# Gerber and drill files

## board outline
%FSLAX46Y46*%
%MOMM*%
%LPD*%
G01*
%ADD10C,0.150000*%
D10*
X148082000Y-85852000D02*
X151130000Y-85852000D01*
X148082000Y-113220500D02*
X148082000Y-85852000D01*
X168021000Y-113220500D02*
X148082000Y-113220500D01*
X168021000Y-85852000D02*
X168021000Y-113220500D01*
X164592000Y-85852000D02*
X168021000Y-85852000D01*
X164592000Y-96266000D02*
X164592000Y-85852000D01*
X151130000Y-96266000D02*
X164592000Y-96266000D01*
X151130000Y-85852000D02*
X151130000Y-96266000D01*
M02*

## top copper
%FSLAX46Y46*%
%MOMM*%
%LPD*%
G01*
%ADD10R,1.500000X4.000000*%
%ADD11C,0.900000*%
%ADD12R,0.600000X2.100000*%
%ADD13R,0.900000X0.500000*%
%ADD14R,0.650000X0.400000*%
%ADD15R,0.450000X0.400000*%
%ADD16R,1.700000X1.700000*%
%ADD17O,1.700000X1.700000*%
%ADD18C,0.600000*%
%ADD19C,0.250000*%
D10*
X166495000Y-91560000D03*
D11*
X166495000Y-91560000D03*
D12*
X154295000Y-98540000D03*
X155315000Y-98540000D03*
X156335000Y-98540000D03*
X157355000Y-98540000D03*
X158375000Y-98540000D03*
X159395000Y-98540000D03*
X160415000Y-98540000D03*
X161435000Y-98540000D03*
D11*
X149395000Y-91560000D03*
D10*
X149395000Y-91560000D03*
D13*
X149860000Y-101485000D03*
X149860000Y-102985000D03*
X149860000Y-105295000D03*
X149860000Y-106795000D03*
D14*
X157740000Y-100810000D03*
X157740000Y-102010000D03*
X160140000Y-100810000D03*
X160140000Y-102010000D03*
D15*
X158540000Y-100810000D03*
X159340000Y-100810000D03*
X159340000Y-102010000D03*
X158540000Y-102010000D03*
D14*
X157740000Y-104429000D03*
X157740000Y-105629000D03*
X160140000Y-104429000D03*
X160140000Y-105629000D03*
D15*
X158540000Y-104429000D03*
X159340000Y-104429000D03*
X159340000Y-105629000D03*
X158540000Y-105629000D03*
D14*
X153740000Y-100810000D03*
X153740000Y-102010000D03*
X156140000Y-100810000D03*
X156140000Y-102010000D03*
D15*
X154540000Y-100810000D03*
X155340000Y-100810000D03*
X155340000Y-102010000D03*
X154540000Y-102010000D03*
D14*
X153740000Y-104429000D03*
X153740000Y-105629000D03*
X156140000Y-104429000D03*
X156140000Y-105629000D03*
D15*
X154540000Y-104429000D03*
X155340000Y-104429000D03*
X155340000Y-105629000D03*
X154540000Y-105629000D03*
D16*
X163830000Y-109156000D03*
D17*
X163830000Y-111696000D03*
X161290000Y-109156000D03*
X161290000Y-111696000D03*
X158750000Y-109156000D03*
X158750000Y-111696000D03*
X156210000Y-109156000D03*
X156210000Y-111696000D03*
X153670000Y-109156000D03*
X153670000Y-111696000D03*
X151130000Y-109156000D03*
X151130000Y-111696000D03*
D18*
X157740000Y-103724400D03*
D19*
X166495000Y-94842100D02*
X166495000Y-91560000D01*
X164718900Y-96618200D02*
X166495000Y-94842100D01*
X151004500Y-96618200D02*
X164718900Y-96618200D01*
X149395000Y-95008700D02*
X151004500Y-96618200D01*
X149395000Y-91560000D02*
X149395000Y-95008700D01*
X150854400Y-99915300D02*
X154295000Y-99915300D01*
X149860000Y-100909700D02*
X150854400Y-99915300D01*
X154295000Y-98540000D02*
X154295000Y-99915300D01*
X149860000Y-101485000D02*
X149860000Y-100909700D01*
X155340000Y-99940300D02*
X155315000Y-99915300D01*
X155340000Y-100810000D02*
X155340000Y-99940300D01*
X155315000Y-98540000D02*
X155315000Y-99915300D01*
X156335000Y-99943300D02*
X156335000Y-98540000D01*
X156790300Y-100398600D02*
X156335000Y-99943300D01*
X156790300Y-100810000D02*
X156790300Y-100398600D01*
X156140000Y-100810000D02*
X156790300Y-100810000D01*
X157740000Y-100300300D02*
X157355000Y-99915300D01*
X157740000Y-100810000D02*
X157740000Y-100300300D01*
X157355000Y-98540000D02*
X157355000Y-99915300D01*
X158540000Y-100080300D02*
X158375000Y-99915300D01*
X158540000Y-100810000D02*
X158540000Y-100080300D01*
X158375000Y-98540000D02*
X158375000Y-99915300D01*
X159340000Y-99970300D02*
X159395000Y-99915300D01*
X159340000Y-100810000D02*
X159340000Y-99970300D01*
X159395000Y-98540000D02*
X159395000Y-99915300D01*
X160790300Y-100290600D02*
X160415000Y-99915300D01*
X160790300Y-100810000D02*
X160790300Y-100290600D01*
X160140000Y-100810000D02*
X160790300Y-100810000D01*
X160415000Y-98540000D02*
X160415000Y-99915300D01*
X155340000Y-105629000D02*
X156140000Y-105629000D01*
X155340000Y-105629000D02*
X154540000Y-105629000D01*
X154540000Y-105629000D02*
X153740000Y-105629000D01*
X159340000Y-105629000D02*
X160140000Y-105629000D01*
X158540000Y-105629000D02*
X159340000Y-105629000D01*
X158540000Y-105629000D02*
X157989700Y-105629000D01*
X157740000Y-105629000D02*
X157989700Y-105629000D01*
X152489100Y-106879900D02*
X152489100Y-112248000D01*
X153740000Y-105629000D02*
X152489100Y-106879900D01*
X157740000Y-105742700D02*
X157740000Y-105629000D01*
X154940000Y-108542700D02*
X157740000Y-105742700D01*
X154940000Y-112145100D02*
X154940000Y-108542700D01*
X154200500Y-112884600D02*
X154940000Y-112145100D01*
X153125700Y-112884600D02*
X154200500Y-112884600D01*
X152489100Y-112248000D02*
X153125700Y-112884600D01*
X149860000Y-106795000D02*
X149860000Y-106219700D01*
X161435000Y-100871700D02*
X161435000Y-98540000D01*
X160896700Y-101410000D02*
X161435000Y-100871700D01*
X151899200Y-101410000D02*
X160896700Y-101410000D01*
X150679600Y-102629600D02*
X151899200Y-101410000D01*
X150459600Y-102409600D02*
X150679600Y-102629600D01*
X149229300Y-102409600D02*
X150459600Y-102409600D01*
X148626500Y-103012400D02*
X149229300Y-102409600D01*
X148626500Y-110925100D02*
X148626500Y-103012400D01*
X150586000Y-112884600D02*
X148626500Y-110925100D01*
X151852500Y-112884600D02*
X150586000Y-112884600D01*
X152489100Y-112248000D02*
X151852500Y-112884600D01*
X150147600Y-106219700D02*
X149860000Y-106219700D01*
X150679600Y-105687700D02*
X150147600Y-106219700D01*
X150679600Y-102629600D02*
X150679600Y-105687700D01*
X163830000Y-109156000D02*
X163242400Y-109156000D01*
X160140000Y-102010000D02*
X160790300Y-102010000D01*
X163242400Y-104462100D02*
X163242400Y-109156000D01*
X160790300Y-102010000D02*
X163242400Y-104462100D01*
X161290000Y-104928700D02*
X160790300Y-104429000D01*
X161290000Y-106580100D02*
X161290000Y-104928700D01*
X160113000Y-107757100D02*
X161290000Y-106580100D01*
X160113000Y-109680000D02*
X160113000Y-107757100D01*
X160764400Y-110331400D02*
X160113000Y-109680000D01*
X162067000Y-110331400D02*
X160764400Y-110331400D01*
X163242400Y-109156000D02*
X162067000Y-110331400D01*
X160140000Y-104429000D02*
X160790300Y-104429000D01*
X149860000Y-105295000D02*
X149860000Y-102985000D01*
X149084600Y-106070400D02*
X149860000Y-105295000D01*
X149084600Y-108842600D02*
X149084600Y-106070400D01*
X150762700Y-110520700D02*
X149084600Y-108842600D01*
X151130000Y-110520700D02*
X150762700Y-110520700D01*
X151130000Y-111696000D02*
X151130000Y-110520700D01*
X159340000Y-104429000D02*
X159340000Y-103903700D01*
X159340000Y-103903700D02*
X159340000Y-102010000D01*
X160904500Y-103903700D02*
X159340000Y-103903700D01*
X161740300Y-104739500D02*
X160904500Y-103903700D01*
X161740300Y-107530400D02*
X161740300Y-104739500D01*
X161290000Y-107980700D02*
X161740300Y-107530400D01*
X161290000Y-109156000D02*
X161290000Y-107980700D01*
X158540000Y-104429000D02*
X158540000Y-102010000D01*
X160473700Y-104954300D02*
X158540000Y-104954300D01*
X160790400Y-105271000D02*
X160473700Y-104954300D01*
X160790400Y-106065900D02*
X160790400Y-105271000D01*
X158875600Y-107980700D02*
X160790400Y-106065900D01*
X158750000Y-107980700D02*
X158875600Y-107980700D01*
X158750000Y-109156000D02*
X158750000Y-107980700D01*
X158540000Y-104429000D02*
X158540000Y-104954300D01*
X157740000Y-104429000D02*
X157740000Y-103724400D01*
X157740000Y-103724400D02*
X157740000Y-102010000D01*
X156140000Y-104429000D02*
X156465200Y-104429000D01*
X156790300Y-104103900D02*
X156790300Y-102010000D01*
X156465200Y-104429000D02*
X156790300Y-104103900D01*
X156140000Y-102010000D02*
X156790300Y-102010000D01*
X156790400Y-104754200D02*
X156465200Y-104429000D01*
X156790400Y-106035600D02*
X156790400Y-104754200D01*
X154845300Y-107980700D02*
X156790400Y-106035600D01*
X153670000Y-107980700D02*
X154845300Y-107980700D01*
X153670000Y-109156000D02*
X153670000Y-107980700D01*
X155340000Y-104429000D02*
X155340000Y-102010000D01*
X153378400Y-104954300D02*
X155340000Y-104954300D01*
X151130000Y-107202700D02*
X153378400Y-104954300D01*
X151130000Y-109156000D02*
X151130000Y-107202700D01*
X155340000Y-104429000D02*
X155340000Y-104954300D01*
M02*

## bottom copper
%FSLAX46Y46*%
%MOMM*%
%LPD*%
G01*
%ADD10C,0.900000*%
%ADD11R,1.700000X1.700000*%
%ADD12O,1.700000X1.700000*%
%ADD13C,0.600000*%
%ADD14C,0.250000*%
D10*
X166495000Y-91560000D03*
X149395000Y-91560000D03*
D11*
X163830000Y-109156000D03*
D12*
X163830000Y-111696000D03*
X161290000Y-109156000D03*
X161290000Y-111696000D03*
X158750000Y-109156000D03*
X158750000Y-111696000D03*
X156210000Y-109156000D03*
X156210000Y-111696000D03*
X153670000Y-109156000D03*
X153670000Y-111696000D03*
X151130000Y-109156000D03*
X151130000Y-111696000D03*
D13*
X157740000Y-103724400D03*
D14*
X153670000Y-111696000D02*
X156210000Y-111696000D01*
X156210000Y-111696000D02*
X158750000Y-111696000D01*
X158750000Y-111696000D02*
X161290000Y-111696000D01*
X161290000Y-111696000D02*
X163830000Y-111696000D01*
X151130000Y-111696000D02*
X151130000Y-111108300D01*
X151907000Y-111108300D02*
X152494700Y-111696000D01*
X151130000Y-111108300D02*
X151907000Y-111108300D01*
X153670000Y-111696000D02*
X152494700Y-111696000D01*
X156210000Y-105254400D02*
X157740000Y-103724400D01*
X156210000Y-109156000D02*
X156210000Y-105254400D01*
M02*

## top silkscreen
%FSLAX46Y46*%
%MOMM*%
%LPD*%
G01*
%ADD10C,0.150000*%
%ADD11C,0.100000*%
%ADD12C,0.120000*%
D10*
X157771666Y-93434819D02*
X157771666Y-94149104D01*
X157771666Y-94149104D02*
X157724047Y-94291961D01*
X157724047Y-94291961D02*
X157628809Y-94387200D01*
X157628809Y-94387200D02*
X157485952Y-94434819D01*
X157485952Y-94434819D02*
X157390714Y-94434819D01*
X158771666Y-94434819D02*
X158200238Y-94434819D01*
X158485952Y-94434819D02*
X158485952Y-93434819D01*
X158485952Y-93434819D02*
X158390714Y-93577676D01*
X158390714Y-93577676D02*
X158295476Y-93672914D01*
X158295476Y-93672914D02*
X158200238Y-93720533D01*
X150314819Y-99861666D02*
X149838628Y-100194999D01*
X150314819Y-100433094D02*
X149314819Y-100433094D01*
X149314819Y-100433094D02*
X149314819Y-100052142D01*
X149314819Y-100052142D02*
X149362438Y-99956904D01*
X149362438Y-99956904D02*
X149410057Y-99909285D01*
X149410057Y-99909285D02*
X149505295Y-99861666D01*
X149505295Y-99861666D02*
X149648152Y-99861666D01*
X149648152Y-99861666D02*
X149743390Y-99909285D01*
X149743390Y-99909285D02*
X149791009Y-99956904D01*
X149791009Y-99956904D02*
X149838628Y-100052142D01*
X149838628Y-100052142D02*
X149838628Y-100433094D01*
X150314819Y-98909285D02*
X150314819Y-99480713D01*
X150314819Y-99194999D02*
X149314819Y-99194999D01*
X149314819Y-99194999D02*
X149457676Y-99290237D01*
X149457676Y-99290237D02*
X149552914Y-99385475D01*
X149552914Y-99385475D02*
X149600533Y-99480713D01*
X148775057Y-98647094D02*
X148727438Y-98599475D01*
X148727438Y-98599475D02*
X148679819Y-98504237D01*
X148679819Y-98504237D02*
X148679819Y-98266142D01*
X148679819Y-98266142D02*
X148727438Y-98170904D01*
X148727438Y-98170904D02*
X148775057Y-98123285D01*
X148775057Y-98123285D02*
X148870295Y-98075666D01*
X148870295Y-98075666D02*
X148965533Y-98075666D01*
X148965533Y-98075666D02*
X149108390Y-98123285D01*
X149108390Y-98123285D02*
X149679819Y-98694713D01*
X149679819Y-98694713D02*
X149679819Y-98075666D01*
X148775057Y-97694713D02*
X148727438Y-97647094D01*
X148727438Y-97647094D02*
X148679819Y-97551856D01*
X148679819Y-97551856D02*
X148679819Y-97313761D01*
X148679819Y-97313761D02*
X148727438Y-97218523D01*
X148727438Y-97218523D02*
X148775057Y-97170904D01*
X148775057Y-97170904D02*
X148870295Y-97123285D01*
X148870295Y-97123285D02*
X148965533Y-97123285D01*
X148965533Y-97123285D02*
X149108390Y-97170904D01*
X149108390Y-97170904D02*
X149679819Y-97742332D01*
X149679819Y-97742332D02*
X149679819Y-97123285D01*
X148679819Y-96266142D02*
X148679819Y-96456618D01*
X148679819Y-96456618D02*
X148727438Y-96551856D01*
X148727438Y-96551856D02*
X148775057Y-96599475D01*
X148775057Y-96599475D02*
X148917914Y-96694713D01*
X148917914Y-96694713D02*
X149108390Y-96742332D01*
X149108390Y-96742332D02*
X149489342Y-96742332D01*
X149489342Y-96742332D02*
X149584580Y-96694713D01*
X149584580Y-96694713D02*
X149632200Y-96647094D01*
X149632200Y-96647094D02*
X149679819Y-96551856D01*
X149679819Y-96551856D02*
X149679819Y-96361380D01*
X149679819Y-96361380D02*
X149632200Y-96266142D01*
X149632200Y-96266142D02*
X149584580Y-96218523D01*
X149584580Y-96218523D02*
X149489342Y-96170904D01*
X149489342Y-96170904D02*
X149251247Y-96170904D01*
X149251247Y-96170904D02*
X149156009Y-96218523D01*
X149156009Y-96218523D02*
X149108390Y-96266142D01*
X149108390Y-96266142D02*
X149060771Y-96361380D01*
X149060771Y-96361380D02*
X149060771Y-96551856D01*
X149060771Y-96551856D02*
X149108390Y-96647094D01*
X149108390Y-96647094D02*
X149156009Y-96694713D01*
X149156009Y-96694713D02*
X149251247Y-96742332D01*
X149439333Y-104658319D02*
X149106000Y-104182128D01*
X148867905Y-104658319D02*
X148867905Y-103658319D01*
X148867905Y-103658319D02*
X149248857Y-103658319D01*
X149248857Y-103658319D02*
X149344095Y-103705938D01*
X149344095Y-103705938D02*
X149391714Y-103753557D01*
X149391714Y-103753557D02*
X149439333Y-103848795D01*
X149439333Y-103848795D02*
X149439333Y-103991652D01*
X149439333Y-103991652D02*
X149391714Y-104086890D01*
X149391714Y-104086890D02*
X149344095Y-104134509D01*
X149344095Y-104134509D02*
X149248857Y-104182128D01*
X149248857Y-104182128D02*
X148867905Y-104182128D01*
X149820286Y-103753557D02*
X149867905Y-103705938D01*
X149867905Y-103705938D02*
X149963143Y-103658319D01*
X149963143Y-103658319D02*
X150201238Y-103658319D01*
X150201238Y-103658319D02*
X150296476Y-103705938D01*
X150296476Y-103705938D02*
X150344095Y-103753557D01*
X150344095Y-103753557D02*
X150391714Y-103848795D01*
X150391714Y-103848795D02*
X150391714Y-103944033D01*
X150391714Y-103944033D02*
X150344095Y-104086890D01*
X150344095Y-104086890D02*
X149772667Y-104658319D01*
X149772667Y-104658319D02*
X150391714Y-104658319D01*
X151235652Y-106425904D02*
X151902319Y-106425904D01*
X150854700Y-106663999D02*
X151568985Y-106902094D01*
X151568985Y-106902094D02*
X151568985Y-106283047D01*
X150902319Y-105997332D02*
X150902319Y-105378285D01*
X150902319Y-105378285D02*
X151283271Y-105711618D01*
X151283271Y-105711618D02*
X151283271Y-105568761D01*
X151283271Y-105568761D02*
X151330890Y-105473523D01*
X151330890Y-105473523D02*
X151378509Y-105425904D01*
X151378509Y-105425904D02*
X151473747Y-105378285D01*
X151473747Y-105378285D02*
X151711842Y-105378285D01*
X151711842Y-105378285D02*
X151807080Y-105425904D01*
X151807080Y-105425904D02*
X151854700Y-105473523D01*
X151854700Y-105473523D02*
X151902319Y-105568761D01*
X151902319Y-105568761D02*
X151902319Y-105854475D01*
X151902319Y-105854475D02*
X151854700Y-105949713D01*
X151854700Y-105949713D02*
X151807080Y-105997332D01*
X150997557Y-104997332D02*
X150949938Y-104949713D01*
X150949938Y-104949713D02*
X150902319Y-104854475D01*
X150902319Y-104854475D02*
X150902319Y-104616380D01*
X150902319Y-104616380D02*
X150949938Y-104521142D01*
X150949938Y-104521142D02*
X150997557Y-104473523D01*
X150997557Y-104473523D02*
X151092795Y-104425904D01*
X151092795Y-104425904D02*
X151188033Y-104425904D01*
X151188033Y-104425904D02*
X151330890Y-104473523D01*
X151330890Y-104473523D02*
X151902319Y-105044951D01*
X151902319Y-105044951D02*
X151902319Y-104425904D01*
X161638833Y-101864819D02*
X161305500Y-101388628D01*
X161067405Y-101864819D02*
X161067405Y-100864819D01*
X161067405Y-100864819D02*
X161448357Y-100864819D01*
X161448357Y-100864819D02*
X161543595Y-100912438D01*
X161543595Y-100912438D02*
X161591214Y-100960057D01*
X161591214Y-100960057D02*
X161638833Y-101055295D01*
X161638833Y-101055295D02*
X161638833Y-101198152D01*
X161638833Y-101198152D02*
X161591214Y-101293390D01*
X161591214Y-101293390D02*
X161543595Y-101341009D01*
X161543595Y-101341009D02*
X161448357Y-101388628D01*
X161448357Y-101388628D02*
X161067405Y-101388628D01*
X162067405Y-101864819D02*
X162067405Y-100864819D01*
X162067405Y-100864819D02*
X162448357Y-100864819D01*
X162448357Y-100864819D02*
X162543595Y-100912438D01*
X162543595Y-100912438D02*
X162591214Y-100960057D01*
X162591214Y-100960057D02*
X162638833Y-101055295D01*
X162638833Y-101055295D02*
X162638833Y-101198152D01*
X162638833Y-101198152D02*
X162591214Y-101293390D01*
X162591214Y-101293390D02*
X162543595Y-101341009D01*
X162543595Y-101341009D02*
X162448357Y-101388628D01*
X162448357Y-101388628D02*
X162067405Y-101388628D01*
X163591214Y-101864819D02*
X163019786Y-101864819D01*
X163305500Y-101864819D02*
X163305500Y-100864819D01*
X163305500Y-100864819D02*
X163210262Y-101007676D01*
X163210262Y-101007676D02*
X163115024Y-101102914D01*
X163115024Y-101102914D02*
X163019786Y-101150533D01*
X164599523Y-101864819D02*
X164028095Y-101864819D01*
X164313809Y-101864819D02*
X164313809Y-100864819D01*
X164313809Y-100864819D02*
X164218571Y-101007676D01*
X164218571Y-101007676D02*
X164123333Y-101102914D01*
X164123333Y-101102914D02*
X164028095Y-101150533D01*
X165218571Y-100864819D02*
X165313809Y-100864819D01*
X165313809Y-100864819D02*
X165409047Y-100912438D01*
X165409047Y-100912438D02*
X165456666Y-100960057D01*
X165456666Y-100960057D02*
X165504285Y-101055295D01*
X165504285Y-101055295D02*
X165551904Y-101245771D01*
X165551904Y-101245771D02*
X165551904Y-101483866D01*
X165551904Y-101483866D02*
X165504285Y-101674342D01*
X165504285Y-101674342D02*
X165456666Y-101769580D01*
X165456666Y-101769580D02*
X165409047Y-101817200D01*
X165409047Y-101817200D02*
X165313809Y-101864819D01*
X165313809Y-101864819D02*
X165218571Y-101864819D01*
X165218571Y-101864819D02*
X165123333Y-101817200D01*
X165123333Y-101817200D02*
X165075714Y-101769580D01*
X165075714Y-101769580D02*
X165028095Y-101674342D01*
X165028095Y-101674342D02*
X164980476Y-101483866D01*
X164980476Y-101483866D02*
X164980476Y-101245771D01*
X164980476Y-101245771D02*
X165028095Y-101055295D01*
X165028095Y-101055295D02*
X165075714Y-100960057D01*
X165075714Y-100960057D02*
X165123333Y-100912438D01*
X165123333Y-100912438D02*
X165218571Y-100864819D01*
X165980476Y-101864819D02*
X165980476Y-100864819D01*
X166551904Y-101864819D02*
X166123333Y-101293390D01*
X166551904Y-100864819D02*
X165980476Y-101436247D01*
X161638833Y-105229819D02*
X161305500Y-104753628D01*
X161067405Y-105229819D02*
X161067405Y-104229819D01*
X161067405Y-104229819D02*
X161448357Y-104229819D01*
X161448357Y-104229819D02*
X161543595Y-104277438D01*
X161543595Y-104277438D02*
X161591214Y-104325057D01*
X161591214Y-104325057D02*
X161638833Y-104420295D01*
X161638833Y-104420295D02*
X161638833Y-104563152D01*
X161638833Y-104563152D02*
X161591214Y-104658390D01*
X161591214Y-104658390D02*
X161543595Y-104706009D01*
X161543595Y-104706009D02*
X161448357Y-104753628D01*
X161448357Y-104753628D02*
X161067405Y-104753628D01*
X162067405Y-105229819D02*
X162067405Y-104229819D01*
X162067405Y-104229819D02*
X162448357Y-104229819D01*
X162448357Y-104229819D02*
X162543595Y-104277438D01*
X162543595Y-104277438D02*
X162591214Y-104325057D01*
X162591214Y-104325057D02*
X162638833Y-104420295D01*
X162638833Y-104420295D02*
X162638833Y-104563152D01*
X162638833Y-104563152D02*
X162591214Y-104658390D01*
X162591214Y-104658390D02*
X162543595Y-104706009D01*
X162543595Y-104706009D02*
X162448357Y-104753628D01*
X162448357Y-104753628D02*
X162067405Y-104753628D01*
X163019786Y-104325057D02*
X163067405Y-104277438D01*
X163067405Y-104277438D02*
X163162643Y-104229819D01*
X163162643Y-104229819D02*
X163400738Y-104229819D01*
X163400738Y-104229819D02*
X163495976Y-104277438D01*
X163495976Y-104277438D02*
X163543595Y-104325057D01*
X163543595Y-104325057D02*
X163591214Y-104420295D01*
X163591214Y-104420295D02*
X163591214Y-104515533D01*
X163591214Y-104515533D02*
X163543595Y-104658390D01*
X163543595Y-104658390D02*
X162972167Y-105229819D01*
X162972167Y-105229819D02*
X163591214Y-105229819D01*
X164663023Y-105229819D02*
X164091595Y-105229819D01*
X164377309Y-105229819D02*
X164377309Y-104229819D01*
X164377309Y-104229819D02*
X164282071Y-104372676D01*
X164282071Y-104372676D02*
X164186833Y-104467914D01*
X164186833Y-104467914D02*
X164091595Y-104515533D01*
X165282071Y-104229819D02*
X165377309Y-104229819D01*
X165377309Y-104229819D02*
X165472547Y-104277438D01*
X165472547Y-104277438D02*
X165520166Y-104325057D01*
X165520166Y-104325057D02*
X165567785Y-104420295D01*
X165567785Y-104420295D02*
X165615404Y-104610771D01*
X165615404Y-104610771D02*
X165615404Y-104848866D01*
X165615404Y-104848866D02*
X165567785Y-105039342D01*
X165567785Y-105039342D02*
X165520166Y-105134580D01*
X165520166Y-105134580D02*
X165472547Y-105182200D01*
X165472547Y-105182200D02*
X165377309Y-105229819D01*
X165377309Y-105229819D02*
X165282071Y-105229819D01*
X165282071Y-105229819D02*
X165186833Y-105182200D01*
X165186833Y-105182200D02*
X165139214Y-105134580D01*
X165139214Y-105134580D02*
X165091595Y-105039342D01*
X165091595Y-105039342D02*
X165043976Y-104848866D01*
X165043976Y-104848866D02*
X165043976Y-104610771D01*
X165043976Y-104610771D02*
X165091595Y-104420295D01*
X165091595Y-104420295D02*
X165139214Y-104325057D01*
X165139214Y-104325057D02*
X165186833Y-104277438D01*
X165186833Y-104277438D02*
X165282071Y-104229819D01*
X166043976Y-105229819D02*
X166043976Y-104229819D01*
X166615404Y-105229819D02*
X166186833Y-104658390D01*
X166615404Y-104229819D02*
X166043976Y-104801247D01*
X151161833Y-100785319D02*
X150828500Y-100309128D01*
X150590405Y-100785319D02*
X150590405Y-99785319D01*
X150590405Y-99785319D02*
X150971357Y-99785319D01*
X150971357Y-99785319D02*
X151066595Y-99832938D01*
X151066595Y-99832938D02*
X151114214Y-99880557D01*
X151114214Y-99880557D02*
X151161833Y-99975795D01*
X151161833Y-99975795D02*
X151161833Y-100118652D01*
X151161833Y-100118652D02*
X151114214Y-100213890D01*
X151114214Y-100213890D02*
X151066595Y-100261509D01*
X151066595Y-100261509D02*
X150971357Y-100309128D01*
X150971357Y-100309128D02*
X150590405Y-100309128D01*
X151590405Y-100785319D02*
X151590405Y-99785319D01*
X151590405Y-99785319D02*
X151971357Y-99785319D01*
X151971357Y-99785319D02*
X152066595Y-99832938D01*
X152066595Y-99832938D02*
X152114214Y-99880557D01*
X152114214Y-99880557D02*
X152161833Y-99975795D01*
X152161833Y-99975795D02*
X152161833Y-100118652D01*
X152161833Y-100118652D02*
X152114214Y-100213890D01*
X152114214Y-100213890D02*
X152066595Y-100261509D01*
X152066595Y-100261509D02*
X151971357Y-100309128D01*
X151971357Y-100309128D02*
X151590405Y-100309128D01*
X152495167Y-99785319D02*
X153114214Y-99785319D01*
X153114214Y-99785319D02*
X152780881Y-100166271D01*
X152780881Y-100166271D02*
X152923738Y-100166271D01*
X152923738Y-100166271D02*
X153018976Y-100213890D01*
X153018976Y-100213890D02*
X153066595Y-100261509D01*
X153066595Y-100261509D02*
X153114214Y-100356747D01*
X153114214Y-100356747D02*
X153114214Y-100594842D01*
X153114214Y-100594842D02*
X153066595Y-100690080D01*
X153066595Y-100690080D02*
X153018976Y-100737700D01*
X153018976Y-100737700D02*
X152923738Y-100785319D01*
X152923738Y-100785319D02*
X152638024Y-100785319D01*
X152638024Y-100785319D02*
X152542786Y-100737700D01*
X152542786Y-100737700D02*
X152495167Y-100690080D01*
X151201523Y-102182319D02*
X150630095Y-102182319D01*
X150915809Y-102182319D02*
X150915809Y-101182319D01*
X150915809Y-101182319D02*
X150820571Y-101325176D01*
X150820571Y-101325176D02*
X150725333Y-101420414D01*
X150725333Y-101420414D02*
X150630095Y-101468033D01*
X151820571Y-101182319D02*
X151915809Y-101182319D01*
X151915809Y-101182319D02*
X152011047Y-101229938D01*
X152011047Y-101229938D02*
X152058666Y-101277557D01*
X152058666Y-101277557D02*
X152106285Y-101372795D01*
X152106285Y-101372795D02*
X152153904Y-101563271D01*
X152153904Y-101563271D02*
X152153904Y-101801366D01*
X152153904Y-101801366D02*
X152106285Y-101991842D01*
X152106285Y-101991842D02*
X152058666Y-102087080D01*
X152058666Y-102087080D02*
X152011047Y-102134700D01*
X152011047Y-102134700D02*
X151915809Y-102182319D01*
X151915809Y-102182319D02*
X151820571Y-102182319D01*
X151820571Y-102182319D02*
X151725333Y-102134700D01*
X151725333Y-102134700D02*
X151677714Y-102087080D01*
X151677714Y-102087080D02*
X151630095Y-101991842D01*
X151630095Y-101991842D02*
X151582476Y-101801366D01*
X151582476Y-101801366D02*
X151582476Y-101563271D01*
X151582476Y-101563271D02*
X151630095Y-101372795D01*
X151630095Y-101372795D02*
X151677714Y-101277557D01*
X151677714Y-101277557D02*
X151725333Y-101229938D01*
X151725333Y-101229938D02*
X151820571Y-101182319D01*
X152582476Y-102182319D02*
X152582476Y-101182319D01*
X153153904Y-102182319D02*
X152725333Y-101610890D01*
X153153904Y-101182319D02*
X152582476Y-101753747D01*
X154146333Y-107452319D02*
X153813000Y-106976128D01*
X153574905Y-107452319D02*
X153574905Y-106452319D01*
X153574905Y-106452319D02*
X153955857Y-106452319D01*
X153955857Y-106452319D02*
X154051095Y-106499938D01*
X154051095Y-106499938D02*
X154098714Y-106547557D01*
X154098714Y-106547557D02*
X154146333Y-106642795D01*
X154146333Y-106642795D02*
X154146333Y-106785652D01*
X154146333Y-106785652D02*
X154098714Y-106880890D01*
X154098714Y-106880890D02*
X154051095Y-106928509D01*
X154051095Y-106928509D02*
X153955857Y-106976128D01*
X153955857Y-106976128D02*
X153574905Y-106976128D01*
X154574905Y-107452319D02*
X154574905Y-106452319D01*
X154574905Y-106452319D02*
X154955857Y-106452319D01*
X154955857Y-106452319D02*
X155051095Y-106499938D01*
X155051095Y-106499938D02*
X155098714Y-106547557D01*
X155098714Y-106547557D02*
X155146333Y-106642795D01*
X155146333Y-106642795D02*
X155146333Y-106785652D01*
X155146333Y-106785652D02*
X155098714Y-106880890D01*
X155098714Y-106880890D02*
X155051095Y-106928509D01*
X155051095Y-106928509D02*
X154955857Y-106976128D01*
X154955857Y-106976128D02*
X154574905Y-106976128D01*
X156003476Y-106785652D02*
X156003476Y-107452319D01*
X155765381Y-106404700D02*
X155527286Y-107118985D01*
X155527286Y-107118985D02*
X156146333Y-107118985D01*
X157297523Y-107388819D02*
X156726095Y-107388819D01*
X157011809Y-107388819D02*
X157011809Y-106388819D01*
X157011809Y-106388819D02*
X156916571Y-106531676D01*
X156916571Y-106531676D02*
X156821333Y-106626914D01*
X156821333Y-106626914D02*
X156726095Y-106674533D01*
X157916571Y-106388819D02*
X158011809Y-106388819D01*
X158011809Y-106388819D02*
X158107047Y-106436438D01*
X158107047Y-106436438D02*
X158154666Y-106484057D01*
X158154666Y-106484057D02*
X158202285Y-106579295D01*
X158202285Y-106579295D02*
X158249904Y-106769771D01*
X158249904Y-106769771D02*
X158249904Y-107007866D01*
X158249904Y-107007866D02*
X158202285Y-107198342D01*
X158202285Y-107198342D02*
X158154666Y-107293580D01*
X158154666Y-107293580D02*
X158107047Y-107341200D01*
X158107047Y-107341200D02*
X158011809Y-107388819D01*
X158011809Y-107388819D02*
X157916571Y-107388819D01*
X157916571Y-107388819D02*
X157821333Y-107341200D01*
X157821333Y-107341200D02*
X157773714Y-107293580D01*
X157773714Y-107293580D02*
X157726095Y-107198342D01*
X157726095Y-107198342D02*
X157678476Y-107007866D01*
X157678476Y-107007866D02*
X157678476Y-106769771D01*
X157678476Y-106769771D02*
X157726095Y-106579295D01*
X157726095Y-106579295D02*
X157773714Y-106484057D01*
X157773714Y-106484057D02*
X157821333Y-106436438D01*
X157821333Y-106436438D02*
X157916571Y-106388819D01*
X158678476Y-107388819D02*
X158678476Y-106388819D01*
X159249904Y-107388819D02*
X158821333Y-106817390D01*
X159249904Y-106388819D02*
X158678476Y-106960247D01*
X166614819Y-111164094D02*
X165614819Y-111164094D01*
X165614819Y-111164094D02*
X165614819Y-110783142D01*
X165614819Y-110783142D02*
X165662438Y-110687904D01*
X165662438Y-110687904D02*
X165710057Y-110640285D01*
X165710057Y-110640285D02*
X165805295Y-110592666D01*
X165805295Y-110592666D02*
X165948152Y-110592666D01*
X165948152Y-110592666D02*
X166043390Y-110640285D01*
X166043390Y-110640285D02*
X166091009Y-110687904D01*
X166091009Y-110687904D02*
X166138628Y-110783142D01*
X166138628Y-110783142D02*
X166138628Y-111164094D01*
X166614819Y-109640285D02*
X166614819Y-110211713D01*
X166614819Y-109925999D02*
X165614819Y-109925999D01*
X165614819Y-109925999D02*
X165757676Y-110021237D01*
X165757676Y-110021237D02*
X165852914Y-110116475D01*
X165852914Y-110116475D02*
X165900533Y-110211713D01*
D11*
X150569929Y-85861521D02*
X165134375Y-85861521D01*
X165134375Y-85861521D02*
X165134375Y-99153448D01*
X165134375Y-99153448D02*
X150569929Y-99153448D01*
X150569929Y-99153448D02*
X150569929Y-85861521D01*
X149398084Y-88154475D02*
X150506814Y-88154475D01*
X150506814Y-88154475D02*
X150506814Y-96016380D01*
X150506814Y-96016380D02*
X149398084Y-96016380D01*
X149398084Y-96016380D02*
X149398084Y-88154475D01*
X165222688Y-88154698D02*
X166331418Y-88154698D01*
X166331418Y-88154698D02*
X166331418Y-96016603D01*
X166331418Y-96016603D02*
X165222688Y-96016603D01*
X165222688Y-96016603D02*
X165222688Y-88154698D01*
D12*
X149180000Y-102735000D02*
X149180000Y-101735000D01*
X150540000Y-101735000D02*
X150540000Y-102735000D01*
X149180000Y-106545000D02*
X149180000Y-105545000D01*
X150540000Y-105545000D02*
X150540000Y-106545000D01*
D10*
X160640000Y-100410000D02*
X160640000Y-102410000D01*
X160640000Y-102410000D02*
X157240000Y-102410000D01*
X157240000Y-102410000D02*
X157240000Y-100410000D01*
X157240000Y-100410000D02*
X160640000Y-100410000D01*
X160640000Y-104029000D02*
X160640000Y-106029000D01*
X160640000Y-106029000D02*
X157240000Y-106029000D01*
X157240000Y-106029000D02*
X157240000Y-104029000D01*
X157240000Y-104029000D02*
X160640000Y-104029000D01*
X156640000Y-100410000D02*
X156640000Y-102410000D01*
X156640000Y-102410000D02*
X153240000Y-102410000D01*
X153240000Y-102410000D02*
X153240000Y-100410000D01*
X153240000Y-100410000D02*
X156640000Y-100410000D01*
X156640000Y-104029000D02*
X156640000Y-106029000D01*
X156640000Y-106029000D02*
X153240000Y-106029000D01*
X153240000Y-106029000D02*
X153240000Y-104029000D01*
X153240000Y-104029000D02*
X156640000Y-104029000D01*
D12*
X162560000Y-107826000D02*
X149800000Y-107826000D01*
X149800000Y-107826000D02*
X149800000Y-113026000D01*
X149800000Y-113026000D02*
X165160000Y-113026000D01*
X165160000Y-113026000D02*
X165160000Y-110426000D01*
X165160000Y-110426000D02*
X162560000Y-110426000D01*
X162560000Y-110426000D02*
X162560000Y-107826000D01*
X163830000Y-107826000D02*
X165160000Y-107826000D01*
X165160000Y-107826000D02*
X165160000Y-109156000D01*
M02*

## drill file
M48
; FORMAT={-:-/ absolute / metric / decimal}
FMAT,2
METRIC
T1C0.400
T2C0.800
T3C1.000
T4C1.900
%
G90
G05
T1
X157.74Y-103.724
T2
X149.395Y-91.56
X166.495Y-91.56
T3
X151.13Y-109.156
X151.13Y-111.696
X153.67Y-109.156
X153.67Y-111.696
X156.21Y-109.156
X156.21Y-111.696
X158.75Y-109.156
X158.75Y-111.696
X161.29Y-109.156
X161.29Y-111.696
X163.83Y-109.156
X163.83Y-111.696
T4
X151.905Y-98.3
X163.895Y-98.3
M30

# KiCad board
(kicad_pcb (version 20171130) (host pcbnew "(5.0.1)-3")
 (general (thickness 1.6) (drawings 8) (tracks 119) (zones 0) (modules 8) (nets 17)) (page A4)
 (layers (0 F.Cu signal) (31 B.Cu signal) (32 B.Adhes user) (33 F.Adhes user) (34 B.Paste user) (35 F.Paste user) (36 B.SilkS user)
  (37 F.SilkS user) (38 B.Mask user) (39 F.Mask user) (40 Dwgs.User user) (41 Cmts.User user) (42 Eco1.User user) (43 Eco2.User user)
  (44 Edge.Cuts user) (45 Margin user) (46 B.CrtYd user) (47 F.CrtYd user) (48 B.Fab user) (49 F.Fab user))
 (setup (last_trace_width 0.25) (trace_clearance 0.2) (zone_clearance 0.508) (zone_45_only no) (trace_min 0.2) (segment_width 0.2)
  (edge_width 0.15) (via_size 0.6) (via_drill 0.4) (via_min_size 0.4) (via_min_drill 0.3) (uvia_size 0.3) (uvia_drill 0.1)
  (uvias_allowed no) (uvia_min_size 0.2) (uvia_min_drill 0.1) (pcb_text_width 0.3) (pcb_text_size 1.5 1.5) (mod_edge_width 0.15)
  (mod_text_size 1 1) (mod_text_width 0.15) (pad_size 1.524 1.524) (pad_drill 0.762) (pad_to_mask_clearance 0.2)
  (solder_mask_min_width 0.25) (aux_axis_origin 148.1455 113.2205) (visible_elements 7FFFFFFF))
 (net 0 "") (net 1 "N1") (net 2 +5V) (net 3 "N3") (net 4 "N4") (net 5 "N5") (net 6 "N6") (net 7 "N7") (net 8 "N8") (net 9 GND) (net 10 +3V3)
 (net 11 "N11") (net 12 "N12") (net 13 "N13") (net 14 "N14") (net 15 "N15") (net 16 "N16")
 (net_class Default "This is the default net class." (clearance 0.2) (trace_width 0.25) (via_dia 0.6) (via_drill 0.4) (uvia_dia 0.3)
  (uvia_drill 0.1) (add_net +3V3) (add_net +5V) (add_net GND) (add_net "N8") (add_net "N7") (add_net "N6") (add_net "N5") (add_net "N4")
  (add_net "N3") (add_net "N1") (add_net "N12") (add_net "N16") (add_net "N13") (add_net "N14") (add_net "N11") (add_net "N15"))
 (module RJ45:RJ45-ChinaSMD (layer F.Cu) (at 150.495 99.06)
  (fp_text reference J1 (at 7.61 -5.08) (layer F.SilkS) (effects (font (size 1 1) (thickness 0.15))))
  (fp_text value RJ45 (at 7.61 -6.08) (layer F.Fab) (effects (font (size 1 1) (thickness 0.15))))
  (fp_line (start 0.074929 -13.198479) (end 14.639375 -13.198479) (layer F.SilkS) (width 0.1))
  (fp_line (start 14.639375 -13.198479) (end 14.639375 0.093448) (layer F.SilkS) (width 0.1))
  (fp_line (start 14.639375 0.093448) (end 0.074929 0.093448) (layer F.SilkS) (width 0.1))
  (fp_line (start 0.074929 0.093448) (end 0.074929 -13.198479) (layer F.SilkS) (width 0.1))
  (fp_line (start -1.096916 -10.905525) (end 0.011814 -10.905525) (layer F.SilkS) (width 0.1))
  (fp_line (start 0.011814 -10.905525) (end 0.011814 -3.04362) (layer F.SilkS) (width 0.1))
  (fp_line (start 0.011814 -3.04362) (end -1.096916 -3.04362) (layer F.SilkS) (width 0.1))
  (fp_line (start -1.096916 -3.04362) (end -1.096916 -10.905525) (layer F.SilkS) (width 0.1))
  (fp_line (start 14.727688 -10.905302) (end 15.836418 -10.905302) (layer F.SilkS) (width 0.1))
  (fp_line (start 15.836418 -10.905302) (end 15.836418 -3.043397) (layer F.SilkS) (width 0.1))
  (fp_line (start 15.836418 -3.043397) (end 14.727688 -3.043397) (layer F.SilkS) (width 0.1))
  (fp_line (start 14.727688 -3.043397) (end 14.727688 -10.905302) (layer F.SilkS) (width 0.1))
  (pad 9 smd rect (at 16 -7.5) (size 1.5 4) (layers F.Cu F.Paste F.Mask) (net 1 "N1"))
  (pad 9 thru_hole circle (at 16 -7.5) (size 0.9 0.9) (drill 0.8) (layers *.Cu *.Mask) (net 1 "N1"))
  (pad "" np_thru_hole circle (at 13.4 -0.76) (size 1.9 1.9) (drill 1.9) (layers *.Cu *.Mask))
  (pad "" np_thru_hole circle (at 1.41 -0.76) (size 1.9 1.9) (drill 1.9) (layers *.Cu *.Mask))
  (pad 8 smd rect (at 3.8 -0.52) (size 0.6 2.1) (layers F.Cu F.Paste F.Mask) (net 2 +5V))
  (pad 7 smd rect (at 4.82 -0.52) (size 0.6 2.1) (layers F.Cu F.Paste F.Mask) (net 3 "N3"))
  (pad 6 smd rect (at 5.84 -0.52) (size 0.6 2.1) (layers F.Cu F.Paste F.Mask) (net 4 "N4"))
  (pad 5 smd rect (at 6.86 -0.52) (size 0.6 2.1) (layers F.Cu F.Paste F.Mask) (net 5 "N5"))
  (pad 4 smd rect (at 7.88 -0.52) (size 0.6 2.1) (layers F.Cu F.Paste F.Mask) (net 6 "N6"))
  (pad 3 smd rect (at 8.9 -0.52) (size 0.6 2.1) (layers F.Cu F.Paste F.Mask) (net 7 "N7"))
  (pad 2 smd rect (at 9.92 -0.52) (size 0.6 2.1) (layers F.Cu F.Paste F.Mask) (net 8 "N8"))
  (pad 1 smd rect (at 10.94 -0.52) (size 0.6 2.1) (layers F.Cu F.Paste F.Mask) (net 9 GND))
  (pad 9 thru_hole circle (at -1.1 -7.5) (size 0.9 0.9) (drill 0.8) (layers *.Cu *.Mask) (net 1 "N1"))
  (pad 9 smd rect (at -1.1 -7.5) (size 1.5 4) (layers F.Cu F.Paste F.Mask) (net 1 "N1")))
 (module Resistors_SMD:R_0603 (layer F.Cu) (at 149.86 102.235 270)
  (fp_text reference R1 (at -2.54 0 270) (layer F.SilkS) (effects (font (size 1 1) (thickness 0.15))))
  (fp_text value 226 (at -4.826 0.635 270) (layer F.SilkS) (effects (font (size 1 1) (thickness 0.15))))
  (fp_line (start 0.5 0.68) (end -0.5 0.68) (layer F.SilkS) (width 0.12))
  (fp_line (start -0.5 -0.68) (end 0.5 -0.68) (layer F.SilkS) (width 0.12))
  (pad 1 smd rect (at -0.75 0 270) (size 0.5 0.9) (layers F.Cu F.Paste F.Mask) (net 2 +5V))
  (pad 2 smd rect (at 0.75 0 270) (size 0.5 0.9) (layers F.Cu F.Paste F.Mask) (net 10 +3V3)))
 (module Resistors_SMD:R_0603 (layer F.Cu) (at 149.86 106.045 270)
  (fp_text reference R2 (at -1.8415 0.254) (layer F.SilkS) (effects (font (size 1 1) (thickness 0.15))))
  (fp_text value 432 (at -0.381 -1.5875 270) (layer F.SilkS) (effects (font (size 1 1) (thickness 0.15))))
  (fp_line (start 0.5 0.68) (end -0.5 0.68) (layer F.SilkS) (width 0.12))
  (fp_line (start -0.5 -0.68) (end 0.5 -0.68) (layer F.SilkS) (width 0.12))
  (pad 1 smd rect (at -0.75 0 270) (size 0.5 0.9) (layers F.Cu F.Paste F.Mask) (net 10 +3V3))
  (pad 2 smd rect (at 0.75 0 270) (size 0.5 0.9) (layers F.Cu F.Paste F.Mask) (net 9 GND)))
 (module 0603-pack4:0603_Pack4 (layer F.Cu) (at 158.94 101.41)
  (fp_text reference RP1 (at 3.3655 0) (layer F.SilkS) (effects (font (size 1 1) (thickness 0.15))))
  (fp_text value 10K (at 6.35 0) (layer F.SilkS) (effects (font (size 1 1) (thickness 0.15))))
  (fp_line (start 1.7 -1) (end 1.7 1) (layer F.SilkS) (width 0.15))
  (fp_line (start 1.7 1) (end -1.7 1) (layer F.SilkS) (width 0.15))
  (fp_line (start -1.7 1) (end -1.7 -1) (layer F.SilkS) (width 0.15))
  (fp_line (start -1.7 -1) (end 1.7 -1) (layer F.SilkS) (width 0.15))
  (pad 1 smd rect (at -1.2 -0.6) (size 0.65 0.4) (layers F.Cu F.Paste F.Mask) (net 5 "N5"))
  (pad 8 smd rect (at -1.2 0.6) (size 0.65 0.4) (layers F.Cu F.Paste F.Mask) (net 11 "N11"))
  (pad 4 smd rect (at 1.2 -0.6) (size 0.65 0.4) (layers F.Cu F.Paste F.Mask) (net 8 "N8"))
  (pad 5 smd rect (at 1.2 0.6) (size 0.65 0.4) (layers F.Cu F.Paste F.Mask) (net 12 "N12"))
  (pad 2 smd rect (at -0.4 -0.6) (size 0.45 0.4) (layers F.Cu F.Paste F.Mask) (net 6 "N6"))
  (pad 3 smd rect (at 0.4 -0.6) (size 0.45 0.4) (layers F.Cu F.Paste F.Mask) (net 7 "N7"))
  (pad 6 smd rect (at 0.4 0.6) (size 0.45 0.4) (layers F.Cu F.Paste F.Mask) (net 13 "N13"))
  (pad 7 smd rect (at -0.4 0.6) (size 0.45 0.4) (layers F.Cu F.Paste F.Mask) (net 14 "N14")))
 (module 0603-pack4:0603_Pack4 (layer F.Cu) (at 158.94 105.029)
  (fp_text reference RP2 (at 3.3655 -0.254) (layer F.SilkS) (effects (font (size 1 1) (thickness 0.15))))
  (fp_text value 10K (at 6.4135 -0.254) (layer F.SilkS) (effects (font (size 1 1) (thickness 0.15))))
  (fp_line (start 1.7 -1) (end 1.7 1) (layer F.SilkS) (width 0.15))
  (fp_line (start 1.7 1) (end -1.7 1) (layer F.SilkS) (width 0.15))
  (fp_line (start -1.7 1) (end -1.7 -1) (layer F.SilkS) (width 0.15))
  (fp_line (start -1.7 -1) (end 1.7 -1) (layer F.SilkS) (width 0.15))
  (pad 1 smd rect (at -1.2 -0.6) (size 0.65 0.4) (layers F.Cu F.Paste F.Mask) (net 11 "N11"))
  (pad 8 smd rect (at -1.2 0.6) (size 0.65 0.4) (layers F.Cu F.Paste F.Mask) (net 9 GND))
  (pad 4 smd rect (at 1.2 -0.6) (size 0.65 0.4) (layers F.Cu F.Paste F.Mask) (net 12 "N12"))
  (pad 5 smd rect (at 1.2 0.6) (size 0.65 0.4) (layers F.Cu F.Paste F.Mask) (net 9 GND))
  (pad 2 smd rect (at -0.4 -0.6) (size 0.45 0.4) (layers F.Cu F.Paste F.Mask) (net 14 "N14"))
  (pad 3 smd rect (at 0.4 -0.6) (size 0.45 0.4) (layers F.Cu F.Paste F.Mask) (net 13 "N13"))
  (pad 6 smd rect (at 0.4 0.6) (size 0.45 0.4) (layers F.Cu F.Paste F.Mask) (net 9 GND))
  (pad 7 smd rect (at -0.4 0.6) (size 0.45 0.4) (layers F.Cu F.Paste F.Mask) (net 9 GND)))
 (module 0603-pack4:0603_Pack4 (layer F.Cu) (at 154.94 101.41)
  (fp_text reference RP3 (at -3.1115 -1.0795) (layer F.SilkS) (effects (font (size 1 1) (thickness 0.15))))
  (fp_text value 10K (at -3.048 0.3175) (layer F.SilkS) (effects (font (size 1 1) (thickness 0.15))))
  (fp_line (start 1.7 -1) (end 1.7 1) (layer F.SilkS) (width 0.15))
  (fp_line (start 1.7 1) (end -1.7 1) (layer F.SilkS) (width 0.15))
  (fp_line (start -1.7 1) (end -1.7 -1) (layer F.SilkS) (width 0.15))
  (fp_line (start -1.7 -1) (end 1.7 -1) (layer F.SilkS) (width 0.15))
  (pad 1 smd rect (at -1.2 -0.6) (size 0.65 0.4) (layers F.Cu F.Paste F.Mask))
  (pad 8 smd rect (at -1.2 0.6) (size 0.65 0.4) (layers F.Cu F.Paste F.Mask))
  (pad 4 smd rect (at 1.2 -0.6) (size 0.65 0.4) (layers F.Cu F.Paste F.Mask) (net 4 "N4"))
  (pad 5 smd rect (at 1.2 0.6) (size 0.65 0.4) (layers F.Cu F.Paste F.Mask) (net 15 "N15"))
  (pad 2 smd rect (at -0.4 -0.6) (size 0.45 0.4) (layers F.Cu F.Paste F.Mask))
  (pad 3 smd rect (at 0.4 -0.6) (size 0.45 0.4) (layers F.Cu F.Paste F.Mask) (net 3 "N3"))
  (pad 6 smd rect (at 0.4 0.6) (size 0.45 0.4) (layers F.Cu F.Paste F.Mask) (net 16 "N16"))
  (pad 7 smd rect (at -0.4 0.6) (size 0.45 0.4) (layers F.Cu F.Paste F.Mask)))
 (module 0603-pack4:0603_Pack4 (layer F.Cu) (at 154.94 105.029)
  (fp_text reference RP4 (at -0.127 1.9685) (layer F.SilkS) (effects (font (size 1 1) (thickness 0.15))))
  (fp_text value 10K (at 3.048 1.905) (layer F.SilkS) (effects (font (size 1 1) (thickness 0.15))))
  (fp_line (start 1.7 -1) (end 1.7 1) (layer F.SilkS) (width 0.15))
  (fp_line (start 1.7 1) (end -1.7 1) (layer F.SilkS) (width 0.15))
  (fp_line (start -1.7 1) (end -1.7 -1) (layer F.SilkS) (width 0.15))
  (fp_line (start -1.7 -1) (end 1.7 -1) (layer F.SilkS) (width 0.15))
  (pad 1 smd rect (at -1.2 -0.6) (size 0.65 0.4) (layers F.Cu F.Paste F.Mask))
  (pad 8 smd rect (at -1.2 0.6) (size 0.65 0.4) (layers F.Cu F.Paste F.Mask) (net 9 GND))
  (pad 4 smd rect (at 1.2 -0.6) (size 0.65 0.4) (layers F.Cu F.Paste F.Mask) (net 15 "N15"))
  (pad 5 smd rect (at 1.2 0.6) (size 0.65 0.4) (layers F.Cu F.Paste F.Mask) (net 9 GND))
  (pad 2 smd rect (at -0.4 -0.6) (size 0.45 0.4) (layers F.Cu F.Paste F.Mask))
  (pad 3 smd rect (at 0.4 -0.6) (size 0.45 0.4) (layers F.Cu F.Paste F.Mask) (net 16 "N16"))
  (pad 6 smd rect (at 0.4 0.6) (size 0.45 0.4) (layers F.Cu F.Paste F.Mask) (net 9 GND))
  (pad 7 smd rect (at -0.4 0.6) (size 0.45 0.4) (layers F.Cu F.Paste F.Mask) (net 9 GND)))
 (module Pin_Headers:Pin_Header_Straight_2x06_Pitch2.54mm (layer F.Cu) (at 163.83 109.156 270)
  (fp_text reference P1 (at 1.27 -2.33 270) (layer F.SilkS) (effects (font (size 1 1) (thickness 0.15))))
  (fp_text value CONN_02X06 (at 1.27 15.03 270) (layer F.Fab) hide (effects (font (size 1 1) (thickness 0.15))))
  (fp_line (start -1.33 1.27) (end -1.33 14.03) (layer F.SilkS) (width 0.12))
  (fp_line (start -1.33 14.03) (end 3.87 14.03) (layer F.SilkS) (width 0.12))
  (fp_line (start 3.87 14.03) (end 3.87 -1.33) (layer F.SilkS) (width 0.12))
  (fp_line (start 3.87 -1.33) (end 1.27 -1.33) (layer F.SilkS) (width 0.12))
  (fp_line (start 1.27 -1.33) (end 1.27 1.27) (layer F.SilkS) (width 0.12))
  (fp_line (start 1.27 1.27) (end -1.33 1.27) (layer F.SilkS) (width 0.12))
  (fp_line (start -1.33 0) (end -1.33 -1.33) (layer F.SilkS) (width 0.12))
  (fp_line (start -1.33 -1.33) (end 0 -1.33) (layer F.SilkS) (width 0.12))
  (pad 1 thru_hole rect (at 0 0 270) (size 1.7 1.7) (drill 1) (layers *.Cu *.Mask) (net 12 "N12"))
  (pad 2 thru_hole oval (at 2.54 0 270) (size 1.7 1.7) (drill 1) (layers *.Cu *.Mask) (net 10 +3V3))
  (pad 3 thru_hole oval (at 0 2.54 270) (size 1.7 1.7) (drill 1) (layers *.Cu *.Mask) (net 13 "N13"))
  (pad 4 thru_hole oval (at 2.54 2.54 270) (size 1.7 1.7) (drill 1) (layers *.Cu *.Mask) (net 10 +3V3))
  (pad 5 thru_hole oval (at 0 5.08 270) (size 1.7 1.7) (drill 1) (layers *.Cu *.Mask) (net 14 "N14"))
  (pad 6 thru_hole oval (at 2.54 5.08 270) (size 1.7 1.7) (drill 1) (layers *.Cu *.Mask) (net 10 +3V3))
  (pad 7 thru_hole oval (at 0 7.62 270) (size 1.7 1.7) (drill 1) (layers *.Cu *.Mask) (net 11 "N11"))
  (pad 8 thru_hole oval (at 2.54 7.62 270) (size 1.7 1.7) (drill 1) (layers *.Cu *.Mask) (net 10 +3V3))
  (pad 9 thru_hole oval (at 0 10.16 270) (size 1.7 1.7) (drill 1) (layers *.Cu *.Mask) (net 15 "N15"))
  (pad 10 thru_hole oval (at 2.54 10.16 270) (size 1.7 1.7) (drill 1) (layers *.Cu *.Mask) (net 10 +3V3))
  (pad 11 thru_hole oval (at 0 12.7 270) (size 1.7 1.7) (drill 1) (layers *.Cu *.Mask) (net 16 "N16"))
  (pad 12 thru_hole oval (at 2.54 12.7 270) (size 1.7 1.7) (drill 1) (layers *.Cu *.Mask) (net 10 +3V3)))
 (gr_line (start 148.082 85.852) (end 151.13 85.852) (angle 90) (layer Edge.Cuts) (width 0.15))
 (gr_line (start 148.082 113.2205) (end 148.082 85.852) (angle 90) (layer Edge.Cuts) (width 0.15))
 (gr_line (start 168.021 113.2205) (end 148.082 113.2205) (angle 90) (layer Edge.Cuts) (width 0.15))
 (gr_line (start 168.021 85.852) (end 168.021 113.2205) (angle 90) (layer Edge.Cuts) (width 0.15))
 (gr_line (start 164.592 85.852) (end 168.021 85.852) (angle 90) (layer Edge.Cuts) (width 0.15))
 (gr_line (start 164.592 96.266) (end 164.592 85.852) (angle 90) (layer Edge.Cuts) (width 0.15))
 (gr_line (start 151.13 96.266) (end 164.592 96.266) (angle 90) (layer Edge.Cuts) (width 0.15))
 (gr_line (start 151.13 85.852) (end 151.13 96.266) (angle 90) (layer Edge.Cuts) (width 0.15))
 (segment (start 166.495 94.8421) (end 166.495 91.56) (width 0.25) (layer F.Cu) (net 1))
 (segment (start 164.7189 96.6182) (end 166.495 94.8421) (width 0.25) (layer F.Cu) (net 1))
 (segment (start 151.0045 96.6182) (end 164.7189 96.6182) (width 0.25) (layer F.Cu) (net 1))
 (segment (start 149.395 95.0087) (end 151.0045 96.6182) (width 0.25) (layer F.Cu) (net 1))
 (segment (start 149.395 91.56) (end 149.395 95.0087) (width 0.25) (layer F.Cu) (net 1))
 (segment (start 150.8544 99.9153) (end 154.295 99.9153) (width 0.25) (layer F.Cu) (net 2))
 (segment (start 149.86 100.9097) (end 150.8544 99.9153) (width 0.25) (layer F.Cu) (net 2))
 (segment (start 154.295 98.54) (end 154.295 99.9153) (width 0.25) (layer F.Cu) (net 2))
 (segment (start 149.86 101.485) (end 149.86 100.9097) (width 0.25) (layer F.Cu) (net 2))
 (segment (start 155.34 99.9403) (end 155.315 99.9153) (width 0.25) (layer F.Cu) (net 3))
 (segment (start 155.34 100.81) (end 155.34 99.9403) (width 0.25) (layer F.Cu) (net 3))
 (segment (start 155.315 98.54) (end 155.315 99.9153) (width 0.25) (layer F.Cu) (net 3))
 (segment (start 156.335 99.9433) (end 156.335 98.54) (width 0.25) (layer F.Cu) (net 4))
 (segment (start 156.7903 100.3986) (end 156.335 99.9433) (width 0.25) (layer F.Cu) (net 4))
 (segment (start 156.7903 100.81) (end 156.7903 100.3986) (width 0.25) (layer F.Cu) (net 4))
 (segment (start 156.14 100.81) (end 156.7903 100.81) (width 0.25) (layer F.Cu) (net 4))
 (segment (start 157.74 100.3003) (end 157.355 99.9153) (width 0.25) (layer F.Cu) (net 5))
 (segment (start 157.74 100.81) (end 157.74 100.3003) (width 0.25) (layer F.Cu) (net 5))
 (segment (start 157.355 98.54) (end 157.355 99.9153) (width 0.25) (layer F.Cu) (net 5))
 (segment (start 158.54 100.0803) (end 158.375 99.9153) (width 0.25) (layer F.Cu) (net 6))
 (segment (start 158.54 100.81) (end 158.54 100.0803) (width 0.25) (layer F.Cu) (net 6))
 (segment (start 158.375 98.54) (end 158.375 99.9153) (width 0.25) (layer F.Cu) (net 6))
 (segment (start 159.34 99.9703) (end 159.395 99.9153) (width 0.25) (layer F.Cu) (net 7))
 (segment (start 159.34 100.81) (end 159.34 99.9703) (width 0.25) (layer F.Cu) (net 7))
 (segment (start 159.395 98.54) (end 159.395 99.9153) (width 0.25) (layer F.Cu) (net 7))
 (segment (start 160.7903 100.2906) (end 160.415 99.9153) (width 0.25) (layer F.Cu) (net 8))
 (segment (start 160.7903 100.81) (end 160.7903 100.2906) (width 0.25) (layer F.Cu) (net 8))
 (segment (start 160.14 100.81) (end 160.7903 100.81) (width 0.25) (layer F.Cu) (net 8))
 (segment (start 160.415 98.54) (end 160.415 99.9153) (width 0.25) (layer F.Cu) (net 8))
 (segment (start 155.34 105.629) (end 156.14 105.629) (width 0.25) (layer F.Cu) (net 9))
 (segment (start 155.34 105.629) (end 154.54 105.629) (width 0.25) (layer F.Cu) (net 9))
 (segment (start 154.54 105.629) (end 153.74 105.629) (width 0.25) (layer F.Cu) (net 9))
 (segment (start 159.34 105.629) (end 160.14 105.629) (width 0.25) (layer F.Cu) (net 9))
 (segment (start 158.54 105.629) (end 159.34 105.629) (width 0.25) (layer F.Cu) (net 9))
 (segment (start 158.54 105.629) (end 157.9897 105.629) (width 0.25) (layer F.Cu) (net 9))
 (segment (start 157.74 105.629) (end 157.9897 105.629) (width 0.25) (layer F.Cu) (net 9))
 (segment (start 152.4891 106.8799) (end 152.4891 112.248) (width 0.25) (layer F.Cu) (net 9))
 (segment (start 153.74 105.629) (end 152.4891 106.8799) (width 0.25) (layer F.Cu) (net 9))
 (segment (start 157.74 105.7427) (end 157.74 105.629) (width 0.25) (layer F.Cu) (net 9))
 (segment (start 154.94 108.5427) (end 157.74 105.7427) (width 0.25) (layer F.Cu) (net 9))
 (segment (start 154.94 112.1451) (end 154.94 108.5427) (width 0.25) (layer F.Cu) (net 9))
 (segment (start 154.2005 112.8846) (end 154.94 112.1451) (width 0.25) (layer F.Cu) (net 9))
 (segment (start 153.1257 112.8846) (end 154.2005 112.8846) (width 0.25) (layer F.Cu) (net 9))
 (segment (start 152.4891 112.248) (end 153.1257 112.8846) (width 0.25) (layer F.Cu) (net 9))
 (segment (start 149.86 106.795) (end 149.86 106.2197) (width 0.25) (layer F.Cu) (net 9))
 (segment (start 161.435 100.8717) (end 161.435 98.54) (width 0.25) (layer F.Cu) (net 9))
 (segment (start 160.8967 101.41) (end 161.435 100.8717) (width 0.25) (layer F.Cu) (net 9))
 (segment (start 151.8992 101.41) (end 160.8967 101.41) (width 0.25) (layer F.Cu) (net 9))
 (segment (start 150.6796 102.6296) (end 151.8992 101.41) (width 0.25) (layer F.Cu) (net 9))
 (segment (start 150.4596 102.4096) (end 150.6796 102.6296) (width 0.25) (layer F.Cu) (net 9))
 (segment (start 149.2293 102.4096) (end 150.4596 102.4096) (width 0.25) (layer F.Cu) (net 9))
 (segment (start 148.6265 103.0124) (end 149.2293 102.4096) (width 0.25) (layer F.Cu) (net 9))
 (segment (start 148.6265 110.9251) (end 148.6265 103.0124) (width 0.25) (layer F.Cu) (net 9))
 (segment (start 150.586 112.8846) (end 148.6265 110.9251) (width 0.25) (layer F.Cu) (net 9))
 (segment (start 151.8525 112.8846) (end 150.586 112.8846) (width 0.25) (layer F.Cu) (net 9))
 (segment (start 152.4891 112.248) (end 151.8525 112.8846) (width 0.25) (layer F.Cu) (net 9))
 (segment (start 150.1476 106.2197) (end 149.86 106.2197) (width 0.25) (layer F.Cu) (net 9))
 (segment (start 150.6796 105.6877) (end 150.1476 106.2197) (width 0.25) (layer F.Cu) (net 9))
 (segment (start 150.6796 102.6296) (end 150.6796 105.6877) (width 0.25) (layer F.Cu) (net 9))
 (segment (start 163.83 109.156) (end 163.2424 109.156) (width 0.25) (layer F.Cu) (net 12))
 (segment (start 160.14 102.01) (end 160.7903 102.01) (width 0.25) (layer F.Cu) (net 12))
 (segment (start 163.2424 104.4621) (end 163.2424 109.156) (width 0.25) (layer F.Cu) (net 12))
 (segment (start 160.7903 102.01) (end 163.2424 104.4621) (width 0.25) (layer F.Cu) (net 12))
 (segment (start 161.29 104.9287) (end 160.7903 104.429) (width 0.25) (layer F.Cu) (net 12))
 (segment (start 161.29 106.5801) (end 161.29 104.9287) (width 0.25) (layer F.Cu) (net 12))
 (segment (start 160.113 107.7571) (end 161.29 106.5801) (width 0.25) (layer F.Cu) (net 12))
 (segment (start 160.113 109.68) (end 160.113 107.7571) (width 0.25) (layer F.Cu) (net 12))
 (segment (start 160.7644 110.3314) (end 160.113 109.68) (width 0.25) (layer F.Cu) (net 12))
 (segment (start 162.067 110.3314) (end 160.7644 110.3314) (width 0.25) (layer F.Cu) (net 12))
 (segment (start 163.2424 109.156) (end 162.067 110.3314) (width 0.25) (layer F.Cu) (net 12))
 (segment (start 160.14 104.429) (end 160.7903 104.429) (width 0.25) (layer F.Cu) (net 12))
 (segment (start 153.67 111.696) (end 156.21 111.696) (width 0.25) (layer B.Cu) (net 10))
 (segment (start 156.21 111.696) (end 158.75 111.696) (width 0.25) (layer B.Cu) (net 10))
 (segment (start 158.75 111.696) (end 161.29 111.696) (width 0.25) (layer B.Cu) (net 10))
 (segment (start 161.29 111.696) (end 163.83 111.696) (width 0.25) (layer B.Cu) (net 10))
 (segment (start 151.13 111.696) (end 151.13 111.1083) (width 0.25) (layer B.Cu) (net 10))
 (segment (start 151.907 111.1083) (end 152.4947 111.696) (width 0.25) (layer B.Cu) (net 10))
 (segment (start 151.13 111.1083) (end 151.907 111.1083) (width 0.25) (layer B.Cu) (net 10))
 (segment (start 153.67 111.696) (end 152.4947 111.696) (width 0.25) (layer B.Cu) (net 10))
 (segment (start 149.86 105.295) (end 149.86 102.985) (width 0.25) (layer F.Cu) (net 10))
 (segment (start 149.0846 106.0704) (end 149.86 105.295) (width 0.25) (layer F.Cu) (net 10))
 (segment (start 149.0846 108.8426) (end 149.0846 106.0704) (width 0.25) (layer F.Cu) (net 10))
 (segment (start 150.7627 110.5207) (end 149.0846 108.8426) (width 0.25) (layer F.Cu) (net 10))
 (segment (start 151.13 110.5207) (end 150.7627 110.5207) (width 0.25) (layer F.Cu) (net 10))
 (segment (start 151.13 111.696) (end 151.13 110.5207) (width 0.25) (layer F.Cu) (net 10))
 (segment (start 159.34 104.429) (end 159.34 103.9037) (width 0.25) (layer F.Cu) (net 13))
 (segment (start 159.34 103.9037) (end 159.34 102.01) (width 0.25) (layer F.Cu) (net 13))
 (segment (start 160.9045 103.9037) (end 159.34 103.9037) (width 0.25) (layer F.Cu) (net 13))
 (segment (start 161.7403 104.7395) (end 160.9045 103.9037) (width 0.25) (layer F.Cu) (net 13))
 (segment (start 161.7403 107.5304) (end 161.7403 104.7395) (width 0.25) (layer F.Cu) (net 13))
 (segment (start 161.29 107.9807) (end 161.7403 107.5304) (width 0.25) (layer F.Cu) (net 13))
 (segment (start 161.29 109.156) (end 161.29 107.9807) (width 0.25) (layer F.Cu) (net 13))
 (segment (start 158.54 104.429) (end 158.54 102.01) (width 0.25) (layer F.Cu) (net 14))
 (segment (start 160.4737 104.9543) (end 158.54 104.9543) (width 0.25) (layer F.Cu) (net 14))
 (segment (start 160.7904 105.271) (end 160.4737 104.9543) (width 0.25) (layer F.Cu) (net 14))
 (segment (start 160.7904 106.0659) (end 160.7904 105.271) (width 0.25) (layer F.Cu) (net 14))
 (segment (start 158.8756 107.9807) (end 160.7904 106.0659) (width 0.25) (layer F.Cu) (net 14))
 (segment (start 158.75 107.9807) (end 158.8756 107.9807) (width 0.25) (layer F.Cu) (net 14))
 (segment (start 158.75 109.156) (end 158.75 107.9807) (width 0.25) (layer F.Cu) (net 14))
 (segment (start 158.54 104.429) (end 158.54 104.9543) (width 0.25) (layer F.Cu) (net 14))
 (via (at 157.74 103.7244) (size 0.6) (layers F.Cu B.Cu) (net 11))
 (segment (start 156.21 105.2544) (end 157.74 103.7244) (width 0.25) (layer B.Cu) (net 11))
 (segment (start 156.21 109.156) (end 156.21 105.2544) (width 0.25) (layer B.Cu) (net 11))
 (segment (start 157.74 104.429) (end 157.74 103.7244) (width 0.25) (layer F.Cu) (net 11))
 (segment (start 157.74 103.7244) (end 157.74 102.01) (width 0.25) (layer F.Cu) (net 11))
 (segment (start 156.14 104.429) (end 156.4652 104.429) (width 0.25) (layer F.Cu) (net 15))
 (segment (start 156.7903 104.1039) (end 156.7903 102.01) (width 0.25) (layer F.Cu) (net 15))
 (segment (start 156.4652 104.429) (end 156.7903 104.1039) (width 0.25) (layer F.Cu) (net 15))
 (segment (start 156.14 102.01) (end 156.7903 102.01) (width 0.25) (layer F.Cu) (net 15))
 (segment (start 156.7904 104.7542) (end 156.4652 104.429) (width 0.25) (layer F.Cu) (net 15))
 (segment (start 156.7904 106.0356) (end 156.7904 104.7542) (width 0.25) (layer F.Cu) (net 15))
 (segment (start 154.8453 107.9807) (end 156.7904 106.0356) (width 0.25) (layer F.Cu) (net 15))
 (segment (start 153.67 107.9807) (end 154.8453 107.9807) (width 0.25) (layer F.Cu) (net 15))
 (segment (start 153.67 109.156) (end 153.67 107.9807) (width 0.25) (layer F.Cu) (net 15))
 (segment (start 155.34 104.429) (end 155.34 102.01) (width 0.25) (layer F.Cu) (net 16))
 (segment (start 153.3784 104.9543) (end 155.34 104.9543) (width 0.25) (layer F.Cu) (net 16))
 (segment (start 151.13 107.2027) (end 153.3784 104.9543) (width 0.25) (layer F.Cu) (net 16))
 (segment (start 151.13 109.156) (end 151.13 107.2027) (width 0.25) (layer F.Cu) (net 16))
 (segment (start 155.34 104.429) (end 155.34 104.9543) (width 0.25) (layer F.Cu) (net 16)))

